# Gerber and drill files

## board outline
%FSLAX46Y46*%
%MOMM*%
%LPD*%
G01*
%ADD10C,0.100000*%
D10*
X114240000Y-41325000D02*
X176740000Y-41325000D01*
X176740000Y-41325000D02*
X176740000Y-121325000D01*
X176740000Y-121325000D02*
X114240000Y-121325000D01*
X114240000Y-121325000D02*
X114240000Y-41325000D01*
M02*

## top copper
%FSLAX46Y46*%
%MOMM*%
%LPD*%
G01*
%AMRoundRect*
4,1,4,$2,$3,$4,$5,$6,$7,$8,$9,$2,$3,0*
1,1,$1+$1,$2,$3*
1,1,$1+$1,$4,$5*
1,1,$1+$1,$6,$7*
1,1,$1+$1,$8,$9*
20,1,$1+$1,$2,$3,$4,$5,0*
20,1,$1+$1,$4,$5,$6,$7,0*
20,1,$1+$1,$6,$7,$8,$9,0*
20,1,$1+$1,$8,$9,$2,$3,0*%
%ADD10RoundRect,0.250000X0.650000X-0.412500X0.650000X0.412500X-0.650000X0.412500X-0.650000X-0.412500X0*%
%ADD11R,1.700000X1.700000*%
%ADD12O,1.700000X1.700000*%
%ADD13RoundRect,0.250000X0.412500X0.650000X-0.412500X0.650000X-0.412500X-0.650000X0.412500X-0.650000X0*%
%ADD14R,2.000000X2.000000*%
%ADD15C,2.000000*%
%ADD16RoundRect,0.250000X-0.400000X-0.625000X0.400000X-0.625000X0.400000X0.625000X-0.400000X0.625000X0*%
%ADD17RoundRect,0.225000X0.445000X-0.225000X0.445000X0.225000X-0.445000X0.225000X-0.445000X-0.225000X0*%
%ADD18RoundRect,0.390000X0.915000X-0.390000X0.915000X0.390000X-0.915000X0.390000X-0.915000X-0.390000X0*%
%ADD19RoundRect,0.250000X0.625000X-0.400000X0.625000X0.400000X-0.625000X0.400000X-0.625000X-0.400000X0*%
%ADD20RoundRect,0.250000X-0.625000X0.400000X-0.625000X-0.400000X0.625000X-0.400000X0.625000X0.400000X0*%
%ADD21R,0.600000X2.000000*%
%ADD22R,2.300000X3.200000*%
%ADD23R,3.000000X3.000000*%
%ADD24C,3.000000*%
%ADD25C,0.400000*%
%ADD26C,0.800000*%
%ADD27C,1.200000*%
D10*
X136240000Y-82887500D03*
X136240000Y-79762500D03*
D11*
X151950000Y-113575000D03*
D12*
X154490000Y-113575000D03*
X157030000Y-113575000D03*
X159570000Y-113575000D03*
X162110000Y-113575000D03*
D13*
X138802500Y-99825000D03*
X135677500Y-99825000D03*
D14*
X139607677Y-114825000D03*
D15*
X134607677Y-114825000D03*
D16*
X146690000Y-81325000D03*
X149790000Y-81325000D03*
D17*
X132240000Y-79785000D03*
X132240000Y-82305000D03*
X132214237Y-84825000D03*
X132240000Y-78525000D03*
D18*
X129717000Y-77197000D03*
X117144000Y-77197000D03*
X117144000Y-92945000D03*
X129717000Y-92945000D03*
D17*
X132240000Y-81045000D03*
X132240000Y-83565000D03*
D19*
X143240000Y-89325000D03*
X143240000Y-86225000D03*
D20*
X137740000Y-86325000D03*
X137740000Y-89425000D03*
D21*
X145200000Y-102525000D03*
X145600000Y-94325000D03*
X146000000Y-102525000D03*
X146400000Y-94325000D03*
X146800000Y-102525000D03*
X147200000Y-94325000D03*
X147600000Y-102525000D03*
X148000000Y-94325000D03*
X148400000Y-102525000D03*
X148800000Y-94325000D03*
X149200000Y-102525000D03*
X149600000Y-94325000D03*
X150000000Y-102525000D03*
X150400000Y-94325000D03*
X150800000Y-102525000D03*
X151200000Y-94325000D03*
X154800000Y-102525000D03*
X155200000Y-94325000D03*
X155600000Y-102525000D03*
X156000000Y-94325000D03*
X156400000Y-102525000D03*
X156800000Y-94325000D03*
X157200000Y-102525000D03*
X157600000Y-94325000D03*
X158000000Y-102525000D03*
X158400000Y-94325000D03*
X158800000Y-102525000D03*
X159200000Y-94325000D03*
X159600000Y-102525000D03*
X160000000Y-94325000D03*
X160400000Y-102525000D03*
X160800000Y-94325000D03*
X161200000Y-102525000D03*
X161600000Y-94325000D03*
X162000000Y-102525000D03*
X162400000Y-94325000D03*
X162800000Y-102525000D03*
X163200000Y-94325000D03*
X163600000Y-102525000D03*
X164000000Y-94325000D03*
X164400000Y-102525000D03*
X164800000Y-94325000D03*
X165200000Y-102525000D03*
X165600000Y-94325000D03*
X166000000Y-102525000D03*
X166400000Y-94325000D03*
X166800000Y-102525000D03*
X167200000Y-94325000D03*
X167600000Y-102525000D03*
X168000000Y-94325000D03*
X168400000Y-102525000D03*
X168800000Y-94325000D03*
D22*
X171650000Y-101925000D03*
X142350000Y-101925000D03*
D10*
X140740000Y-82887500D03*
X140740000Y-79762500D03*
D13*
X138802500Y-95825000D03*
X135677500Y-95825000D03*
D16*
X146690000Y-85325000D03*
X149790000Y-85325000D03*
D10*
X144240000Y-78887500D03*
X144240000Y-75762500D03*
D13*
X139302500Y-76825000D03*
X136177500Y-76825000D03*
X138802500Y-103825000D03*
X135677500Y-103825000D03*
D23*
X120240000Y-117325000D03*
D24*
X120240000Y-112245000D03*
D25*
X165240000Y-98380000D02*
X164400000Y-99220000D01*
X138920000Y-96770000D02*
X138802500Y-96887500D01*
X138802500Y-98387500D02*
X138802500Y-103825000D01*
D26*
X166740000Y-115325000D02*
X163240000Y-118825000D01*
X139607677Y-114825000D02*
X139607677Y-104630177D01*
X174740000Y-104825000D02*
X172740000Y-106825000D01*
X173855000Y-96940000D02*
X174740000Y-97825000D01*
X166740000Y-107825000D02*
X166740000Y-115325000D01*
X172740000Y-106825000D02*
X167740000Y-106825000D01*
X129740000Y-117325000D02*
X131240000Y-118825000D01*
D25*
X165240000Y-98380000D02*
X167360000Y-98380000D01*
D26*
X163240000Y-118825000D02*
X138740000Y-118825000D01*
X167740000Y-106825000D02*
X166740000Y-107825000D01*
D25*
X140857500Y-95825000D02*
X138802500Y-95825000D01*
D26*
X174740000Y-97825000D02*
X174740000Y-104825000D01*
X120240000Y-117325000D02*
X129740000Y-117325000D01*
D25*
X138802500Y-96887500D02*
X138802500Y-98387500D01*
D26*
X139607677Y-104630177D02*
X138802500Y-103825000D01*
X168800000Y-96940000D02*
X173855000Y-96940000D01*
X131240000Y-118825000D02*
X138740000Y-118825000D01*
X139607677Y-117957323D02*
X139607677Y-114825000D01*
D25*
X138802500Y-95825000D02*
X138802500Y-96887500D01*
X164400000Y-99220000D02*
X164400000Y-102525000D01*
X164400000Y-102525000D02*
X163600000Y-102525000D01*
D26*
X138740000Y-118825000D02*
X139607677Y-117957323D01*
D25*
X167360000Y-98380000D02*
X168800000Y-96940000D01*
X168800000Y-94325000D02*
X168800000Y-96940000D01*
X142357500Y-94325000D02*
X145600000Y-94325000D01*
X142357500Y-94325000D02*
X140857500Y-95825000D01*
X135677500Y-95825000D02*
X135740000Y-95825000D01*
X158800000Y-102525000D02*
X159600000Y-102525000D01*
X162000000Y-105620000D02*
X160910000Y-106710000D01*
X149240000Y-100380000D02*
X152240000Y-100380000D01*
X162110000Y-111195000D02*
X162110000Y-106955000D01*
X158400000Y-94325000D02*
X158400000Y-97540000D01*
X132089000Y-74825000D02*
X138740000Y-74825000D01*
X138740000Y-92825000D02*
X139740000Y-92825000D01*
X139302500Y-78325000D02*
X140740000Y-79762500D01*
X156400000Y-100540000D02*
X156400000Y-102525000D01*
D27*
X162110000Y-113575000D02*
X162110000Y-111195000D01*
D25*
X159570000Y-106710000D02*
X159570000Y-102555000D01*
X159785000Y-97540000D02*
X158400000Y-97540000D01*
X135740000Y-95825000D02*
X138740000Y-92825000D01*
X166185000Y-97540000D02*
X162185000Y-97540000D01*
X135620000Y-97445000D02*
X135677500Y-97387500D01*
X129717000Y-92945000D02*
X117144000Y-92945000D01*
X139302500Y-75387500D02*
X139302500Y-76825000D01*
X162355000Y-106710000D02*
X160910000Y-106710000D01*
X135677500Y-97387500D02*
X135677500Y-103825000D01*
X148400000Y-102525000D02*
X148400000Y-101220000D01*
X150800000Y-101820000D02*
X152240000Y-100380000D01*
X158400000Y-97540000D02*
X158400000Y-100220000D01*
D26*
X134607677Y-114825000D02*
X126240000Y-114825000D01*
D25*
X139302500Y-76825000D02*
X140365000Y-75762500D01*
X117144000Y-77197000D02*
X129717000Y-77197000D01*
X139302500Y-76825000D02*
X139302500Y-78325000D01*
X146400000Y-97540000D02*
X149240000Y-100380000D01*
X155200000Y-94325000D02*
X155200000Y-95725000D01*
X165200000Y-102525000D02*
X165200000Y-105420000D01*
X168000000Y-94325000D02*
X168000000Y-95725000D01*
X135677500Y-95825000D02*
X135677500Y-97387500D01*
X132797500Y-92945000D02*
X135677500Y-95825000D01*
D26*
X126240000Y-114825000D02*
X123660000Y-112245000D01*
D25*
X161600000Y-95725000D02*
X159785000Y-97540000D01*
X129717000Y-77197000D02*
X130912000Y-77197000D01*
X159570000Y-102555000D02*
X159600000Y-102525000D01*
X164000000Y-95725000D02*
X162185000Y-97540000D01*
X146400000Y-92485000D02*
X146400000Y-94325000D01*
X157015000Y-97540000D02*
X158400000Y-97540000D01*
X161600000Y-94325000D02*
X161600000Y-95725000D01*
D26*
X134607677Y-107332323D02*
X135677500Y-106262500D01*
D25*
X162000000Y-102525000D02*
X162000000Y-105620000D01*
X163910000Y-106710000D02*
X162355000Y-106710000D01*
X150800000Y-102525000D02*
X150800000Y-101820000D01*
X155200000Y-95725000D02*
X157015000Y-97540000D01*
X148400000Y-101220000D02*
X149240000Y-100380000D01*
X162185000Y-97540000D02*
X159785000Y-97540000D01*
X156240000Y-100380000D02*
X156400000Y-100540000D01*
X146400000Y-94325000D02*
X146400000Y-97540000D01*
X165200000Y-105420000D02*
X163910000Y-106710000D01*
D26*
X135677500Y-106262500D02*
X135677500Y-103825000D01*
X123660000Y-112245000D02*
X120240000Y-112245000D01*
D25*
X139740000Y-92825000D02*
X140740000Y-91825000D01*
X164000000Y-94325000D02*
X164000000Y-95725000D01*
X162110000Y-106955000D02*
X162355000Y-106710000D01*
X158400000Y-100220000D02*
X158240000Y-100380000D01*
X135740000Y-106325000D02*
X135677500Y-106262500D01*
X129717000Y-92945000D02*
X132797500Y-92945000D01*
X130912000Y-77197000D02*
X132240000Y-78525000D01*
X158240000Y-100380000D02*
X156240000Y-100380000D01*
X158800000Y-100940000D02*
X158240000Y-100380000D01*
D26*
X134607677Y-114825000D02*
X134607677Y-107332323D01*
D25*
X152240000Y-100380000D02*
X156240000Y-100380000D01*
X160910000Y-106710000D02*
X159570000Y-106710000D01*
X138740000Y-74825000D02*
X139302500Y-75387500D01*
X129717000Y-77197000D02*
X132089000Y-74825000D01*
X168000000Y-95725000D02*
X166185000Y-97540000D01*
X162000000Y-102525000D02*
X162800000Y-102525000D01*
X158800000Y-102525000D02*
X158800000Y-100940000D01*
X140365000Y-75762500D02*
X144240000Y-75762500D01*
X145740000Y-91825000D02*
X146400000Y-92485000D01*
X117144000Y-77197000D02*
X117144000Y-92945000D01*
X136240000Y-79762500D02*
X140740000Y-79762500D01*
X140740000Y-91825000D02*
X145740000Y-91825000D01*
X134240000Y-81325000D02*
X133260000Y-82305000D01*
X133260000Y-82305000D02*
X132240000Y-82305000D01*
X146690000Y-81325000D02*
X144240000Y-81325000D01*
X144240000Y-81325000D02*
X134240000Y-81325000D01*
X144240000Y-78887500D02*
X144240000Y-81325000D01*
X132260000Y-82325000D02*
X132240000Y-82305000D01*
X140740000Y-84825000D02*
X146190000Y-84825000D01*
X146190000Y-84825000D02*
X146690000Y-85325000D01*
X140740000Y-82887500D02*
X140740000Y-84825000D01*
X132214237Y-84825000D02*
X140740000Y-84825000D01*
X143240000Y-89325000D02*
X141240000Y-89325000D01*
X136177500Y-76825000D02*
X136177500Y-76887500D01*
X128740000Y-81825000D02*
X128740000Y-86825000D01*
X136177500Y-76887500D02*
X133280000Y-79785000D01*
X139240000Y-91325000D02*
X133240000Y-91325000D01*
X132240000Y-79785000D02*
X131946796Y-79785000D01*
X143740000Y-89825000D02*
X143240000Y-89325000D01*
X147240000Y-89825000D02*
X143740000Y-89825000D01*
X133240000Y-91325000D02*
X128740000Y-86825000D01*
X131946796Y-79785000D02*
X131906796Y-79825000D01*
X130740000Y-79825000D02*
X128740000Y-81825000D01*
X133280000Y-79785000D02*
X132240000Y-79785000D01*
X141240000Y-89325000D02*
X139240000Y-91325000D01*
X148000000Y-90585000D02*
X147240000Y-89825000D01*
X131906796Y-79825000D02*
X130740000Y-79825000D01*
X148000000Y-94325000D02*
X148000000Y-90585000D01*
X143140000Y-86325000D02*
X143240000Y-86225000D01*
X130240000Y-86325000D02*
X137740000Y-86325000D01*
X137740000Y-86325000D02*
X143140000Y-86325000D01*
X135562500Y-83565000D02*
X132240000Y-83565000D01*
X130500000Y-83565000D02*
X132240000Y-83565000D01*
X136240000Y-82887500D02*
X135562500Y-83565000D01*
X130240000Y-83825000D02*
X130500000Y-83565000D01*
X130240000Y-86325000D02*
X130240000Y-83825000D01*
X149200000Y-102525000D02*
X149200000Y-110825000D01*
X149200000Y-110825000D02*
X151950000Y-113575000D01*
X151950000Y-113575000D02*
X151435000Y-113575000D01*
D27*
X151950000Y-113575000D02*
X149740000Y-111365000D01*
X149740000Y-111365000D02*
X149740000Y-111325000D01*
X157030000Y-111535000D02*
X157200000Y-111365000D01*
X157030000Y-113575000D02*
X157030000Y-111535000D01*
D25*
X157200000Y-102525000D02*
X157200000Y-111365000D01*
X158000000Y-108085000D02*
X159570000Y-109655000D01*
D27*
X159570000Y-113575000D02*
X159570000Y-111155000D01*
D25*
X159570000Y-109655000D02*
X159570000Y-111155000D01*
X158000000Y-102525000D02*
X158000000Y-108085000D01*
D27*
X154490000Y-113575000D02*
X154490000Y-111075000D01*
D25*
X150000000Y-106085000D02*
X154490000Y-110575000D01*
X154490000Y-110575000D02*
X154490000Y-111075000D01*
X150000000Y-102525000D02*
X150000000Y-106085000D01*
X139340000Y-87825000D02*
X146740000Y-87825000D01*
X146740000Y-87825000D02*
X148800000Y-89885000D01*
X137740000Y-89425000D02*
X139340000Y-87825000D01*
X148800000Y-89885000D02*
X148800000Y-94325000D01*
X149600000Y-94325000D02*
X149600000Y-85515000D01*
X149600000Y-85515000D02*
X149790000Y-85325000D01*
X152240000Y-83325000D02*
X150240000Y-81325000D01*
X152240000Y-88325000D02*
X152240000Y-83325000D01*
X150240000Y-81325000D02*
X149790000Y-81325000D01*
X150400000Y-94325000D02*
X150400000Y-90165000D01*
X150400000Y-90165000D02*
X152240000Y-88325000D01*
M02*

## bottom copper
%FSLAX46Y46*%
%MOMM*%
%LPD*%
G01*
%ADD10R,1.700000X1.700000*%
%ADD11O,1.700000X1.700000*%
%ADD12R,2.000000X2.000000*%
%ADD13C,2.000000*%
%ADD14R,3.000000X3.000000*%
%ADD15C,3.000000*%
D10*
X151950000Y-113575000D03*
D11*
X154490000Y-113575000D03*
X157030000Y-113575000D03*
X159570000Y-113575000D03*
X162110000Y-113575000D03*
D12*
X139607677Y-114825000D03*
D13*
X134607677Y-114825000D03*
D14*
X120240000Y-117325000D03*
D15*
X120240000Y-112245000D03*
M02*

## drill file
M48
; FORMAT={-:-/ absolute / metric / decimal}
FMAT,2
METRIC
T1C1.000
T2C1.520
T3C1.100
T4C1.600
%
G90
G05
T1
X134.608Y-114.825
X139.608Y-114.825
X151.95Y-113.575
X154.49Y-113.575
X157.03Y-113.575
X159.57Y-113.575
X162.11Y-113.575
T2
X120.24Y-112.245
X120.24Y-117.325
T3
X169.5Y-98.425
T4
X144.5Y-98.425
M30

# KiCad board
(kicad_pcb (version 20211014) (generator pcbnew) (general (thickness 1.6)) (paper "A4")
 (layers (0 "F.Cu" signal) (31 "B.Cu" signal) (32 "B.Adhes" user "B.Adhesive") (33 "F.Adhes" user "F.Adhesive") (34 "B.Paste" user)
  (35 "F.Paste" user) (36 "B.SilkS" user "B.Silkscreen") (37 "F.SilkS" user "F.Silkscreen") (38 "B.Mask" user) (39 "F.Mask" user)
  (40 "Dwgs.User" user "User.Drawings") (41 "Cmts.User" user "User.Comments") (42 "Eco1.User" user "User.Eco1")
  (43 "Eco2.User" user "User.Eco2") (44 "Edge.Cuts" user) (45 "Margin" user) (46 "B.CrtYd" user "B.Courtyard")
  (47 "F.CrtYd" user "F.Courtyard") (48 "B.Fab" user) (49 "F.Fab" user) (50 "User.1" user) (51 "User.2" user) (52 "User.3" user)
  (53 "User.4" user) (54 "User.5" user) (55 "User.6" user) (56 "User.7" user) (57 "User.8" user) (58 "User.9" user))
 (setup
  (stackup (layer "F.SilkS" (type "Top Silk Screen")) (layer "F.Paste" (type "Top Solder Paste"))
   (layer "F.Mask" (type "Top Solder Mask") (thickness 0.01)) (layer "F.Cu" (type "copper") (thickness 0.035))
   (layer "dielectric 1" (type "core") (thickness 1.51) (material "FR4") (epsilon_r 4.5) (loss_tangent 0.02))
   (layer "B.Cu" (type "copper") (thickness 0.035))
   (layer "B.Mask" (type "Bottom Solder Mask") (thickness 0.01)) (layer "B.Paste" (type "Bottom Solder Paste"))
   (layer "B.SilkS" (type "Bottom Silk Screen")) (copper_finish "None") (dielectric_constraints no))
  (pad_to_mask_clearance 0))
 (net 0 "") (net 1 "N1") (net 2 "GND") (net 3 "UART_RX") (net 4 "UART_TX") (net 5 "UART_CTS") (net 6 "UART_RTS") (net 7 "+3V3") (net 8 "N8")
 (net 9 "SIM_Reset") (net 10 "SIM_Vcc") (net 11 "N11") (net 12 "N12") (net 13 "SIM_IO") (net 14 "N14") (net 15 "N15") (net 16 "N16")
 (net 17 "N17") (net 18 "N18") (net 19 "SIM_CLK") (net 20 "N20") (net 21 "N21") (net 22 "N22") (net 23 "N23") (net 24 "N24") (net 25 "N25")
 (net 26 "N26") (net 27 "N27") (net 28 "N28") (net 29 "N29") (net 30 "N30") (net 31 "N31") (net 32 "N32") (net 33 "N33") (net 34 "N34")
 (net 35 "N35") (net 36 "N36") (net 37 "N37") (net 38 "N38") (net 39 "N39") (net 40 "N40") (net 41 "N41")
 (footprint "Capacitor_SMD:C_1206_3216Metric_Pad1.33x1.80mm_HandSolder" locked (layer "F.Cu") (at 136.24 81.325 90)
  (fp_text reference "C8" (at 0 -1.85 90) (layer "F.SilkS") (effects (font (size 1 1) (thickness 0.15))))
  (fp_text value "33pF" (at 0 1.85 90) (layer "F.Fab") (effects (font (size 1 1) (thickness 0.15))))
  (pad "1" smd roundrect locked (at -1.5625 0 90) (size 1.325 1.8) (layers "F.Cu" "F.Paste" "F.Mask") (roundrect_rratio 0.188679)
   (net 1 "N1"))
  (pad "2" smd roundrect locked (at 1.5625 0 90) (size 1.325 1.8) (layers "F.Cu" "F.Paste" "F.Mask") (roundrect_rratio 0.188679)
   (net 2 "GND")))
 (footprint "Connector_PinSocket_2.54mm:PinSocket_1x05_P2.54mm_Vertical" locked (layer "F.Cu") (at 151.95 113.575 90)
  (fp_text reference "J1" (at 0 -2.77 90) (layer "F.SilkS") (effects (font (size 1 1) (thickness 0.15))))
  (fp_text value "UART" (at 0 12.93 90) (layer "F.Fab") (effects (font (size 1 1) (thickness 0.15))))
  (pad "1" thru_hole rect locked (at 0 0 90) (size 1.7 1.7) (drill 1) (layers *.Cu *.Mask) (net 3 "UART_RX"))
  (pad "2" thru_hole oval locked (at 0 2.54 90) (size 1.7 1.7) (drill 1) (layers *.Cu *.Mask) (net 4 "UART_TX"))
  (pad "3" thru_hole oval locked (at 0 5.08 90) (size 1.7 1.7) (drill 1) (layers *.Cu *.Mask) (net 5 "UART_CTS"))
  (pad "4" thru_hole oval locked (at 0 7.62 90) (size 1.7 1.7) (drill 1) (layers *.Cu *.Mask) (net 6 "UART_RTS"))
  (pad "5" thru_hole oval locked (at 0 10.16 90) (size 1.7 1.7) (drill 1) (layers *.Cu *.Mask) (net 2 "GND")))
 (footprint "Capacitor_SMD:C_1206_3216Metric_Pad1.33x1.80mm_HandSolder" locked (layer "F.Cu") (at 137.24 99.825 180)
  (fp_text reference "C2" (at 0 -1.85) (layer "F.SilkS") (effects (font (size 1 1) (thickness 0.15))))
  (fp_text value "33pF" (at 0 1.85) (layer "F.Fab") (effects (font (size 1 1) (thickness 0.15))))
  (pad "1" smd roundrect locked (at -1.5625 0 180) (size 1.325 1.8) (layers "F.Cu" "F.Paste" "F.Mask") (roundrect_rratio 0.188679)
   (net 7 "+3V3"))
  (pad "2" smd roundrect locked (at 1.5625 0 180) (size 1.325 1.8) (layers "F.Cu" "F.Paste" "F.Mask") (roundrect_rratio 0.188679)
   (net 2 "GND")))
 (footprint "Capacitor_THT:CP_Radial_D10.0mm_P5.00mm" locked (layer "F.Cu") (at 139.607677 114.825 180)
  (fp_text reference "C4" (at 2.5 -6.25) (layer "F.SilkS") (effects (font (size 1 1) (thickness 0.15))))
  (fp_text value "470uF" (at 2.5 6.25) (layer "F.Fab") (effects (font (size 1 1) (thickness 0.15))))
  (pad "1" thru_hole rect locked (at 0 0 180) (size 2 2) (drill 1) (layers *.Cu *.Mask) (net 7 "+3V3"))
  (pad "2" thru_hole circle locked (at 5 0 180) (size 2 2) (drill 1) (layers *.Cu *.Mask) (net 2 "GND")))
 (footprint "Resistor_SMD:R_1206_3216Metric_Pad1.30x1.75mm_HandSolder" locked (layer "F.Cu") (at 148.24 81.325)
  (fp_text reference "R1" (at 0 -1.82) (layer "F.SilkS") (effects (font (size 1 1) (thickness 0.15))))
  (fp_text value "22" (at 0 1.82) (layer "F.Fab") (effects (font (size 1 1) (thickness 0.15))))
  (pad "1" smd roundrect locked (at -1.55 0) (size 1.3 1.75) (layers "F.Cu" "F.Paste" "F.Mask") (roundrect_rratio 0.192308) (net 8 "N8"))
  (pad "2" smd roundrect locked (at 1.55 0) (size 1.3 1.75) (layers "F.Cu" "F.Paste" "F.Mask") (roundrect_rratio 0.192308)
   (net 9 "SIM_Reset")))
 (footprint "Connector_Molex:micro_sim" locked (layer "F.Cu") (at 123.24 85.325 -90)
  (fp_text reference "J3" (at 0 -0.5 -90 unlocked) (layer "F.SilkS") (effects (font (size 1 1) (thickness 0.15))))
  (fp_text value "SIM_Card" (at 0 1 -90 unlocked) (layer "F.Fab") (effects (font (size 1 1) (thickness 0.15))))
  (pad "1" smd roundrect locked (at -5.54 -9 90) (size 0.9 1.34) (layers "F.Cu" "F.Paste" "F.Mask") (roundrect_rratio 0.25)
   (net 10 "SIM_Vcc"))
  (pad "2" smd roundrect locked (at -3.02 -9 90) (size 0.9 1.34) (layers "F.Cu" "F.Paste" "F.Mask") (roundrect_rratio 0.25) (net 8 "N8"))
  (pad "3" smd roundrect locked (at -0.5 -8.974237 90) (size 0.9 1.34) (layers "F.Cu" "F.Paste" "F.Mask") (roundrect_rratio 0.25)
   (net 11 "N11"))
  (pad "5" smd roundrect locked (at -6.8 -9 90) (size 0.9 1.34) (layers "F.Cu" "F.Paste" "F.Mask") (roundrect_rratio 0.25) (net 2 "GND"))
  (pad "5" smd roundrect locked (at -8.128 -6.477 90) (size 1.56 2.61) (layers "F.Cu" "F.Paste" "F.Mask") (roundrect_rratio 0.25)
   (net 2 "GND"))
  (pad "5" smd roundrect locked (at -8.128 6.096 90) (size 1.56 2.61) (layers "F.Cu" "F.Paste" "F.Mask") (roundrect_rratio 0.25)
   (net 2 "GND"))
  (pad "5" smd roundrect locked (at 7.62 6.096 90) (size 1.56 2.61) (layers "F.Cu" "F.Paste" "F.Mask") (roundrect_rratio 0.25) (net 2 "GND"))
  (pad "5" smd roundrect locked (at 7.62 -6.477 90) (size 1.56 2.61) (layers "F.Cu" "F.Paste" "F.Mask") (roundrect_rratio 0.25)
   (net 2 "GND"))
  (pad "6" smd roundrect locked (at -4.28 -9 90) (size 0.9 1.34) (layers "F.Cu" "F.Paste" "F.Mask") (roundrect_rratio 0.25) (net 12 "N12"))
  (pad "7" smd roundrect locked (at -1.76 -9 90) (size 0.9 1.34) (layers "F.Cu" "F.Paste" "F.Mask") (roundrect_rratio 0.25) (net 1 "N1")))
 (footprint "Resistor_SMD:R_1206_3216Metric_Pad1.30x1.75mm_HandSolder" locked (layer "F.Cu") (at 143.24 87.775 90)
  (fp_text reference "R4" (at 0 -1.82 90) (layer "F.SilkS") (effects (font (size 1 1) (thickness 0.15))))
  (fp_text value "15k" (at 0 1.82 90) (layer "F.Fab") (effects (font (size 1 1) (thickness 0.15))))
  (pad "1" smd roundrect locked (at -1.55 0 90) (size 1.3 1.75) (layers "F.Cu" "F.Paste" "F.Mask") (roundrect_rratio 0.192308)
   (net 10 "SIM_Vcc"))
  (pad "2" smd roundrect locked (at 1.55 0 90) (size 1.3 1.75) (layers "F.Cu" "F.Paste" "F.Mask") (roundrect_rratio 0.192308) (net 1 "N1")))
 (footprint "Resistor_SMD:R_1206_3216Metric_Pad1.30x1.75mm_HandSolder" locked (layer "F.Cu") (at 137.74 87.875 -90)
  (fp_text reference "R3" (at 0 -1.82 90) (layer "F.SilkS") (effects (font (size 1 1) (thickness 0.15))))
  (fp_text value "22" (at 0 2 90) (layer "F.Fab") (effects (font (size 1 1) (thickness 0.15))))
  (pad "1" smd roundrect locked (at -1.55 0 270) (size 1.3 1.75) (layers "F.Cu" "F.Paste" "F.Mask") (roundrect_rratio 0.192308) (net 1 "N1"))
  (pad "2" smd roundrect locked (at 1.55 0 270) (size 1.3 1.75) (layers "F.Cu" "F.Paste" "F.Mask") (roundrect_rratio 0.192308)
   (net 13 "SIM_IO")))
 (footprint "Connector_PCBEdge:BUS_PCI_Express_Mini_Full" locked (layer "F.Cu") (at 157 98.425)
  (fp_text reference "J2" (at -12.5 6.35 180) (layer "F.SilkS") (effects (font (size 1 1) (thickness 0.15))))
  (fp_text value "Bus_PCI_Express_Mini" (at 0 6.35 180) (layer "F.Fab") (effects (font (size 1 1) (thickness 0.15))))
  (pad "" np_thru_hole circle locked (at -12.5 0) (size 1.6 1.6) (drill 1.6) (layers *.Cu *.Mask))
  (pad "" np_thru_hole circle locked (at 12.5 0) (size 1.1 1.1) (drill 1.1) (layers *.Cu *.Mask))
  (pad "1" smd rect locked (at -11.8 4.1) (size 0.6 2) (layers "F.Cu" "F.Paste" "F.Mask") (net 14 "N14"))
  (pad "2" smd rect locked (at -11.4 -4.1) (size 0.6 2) (layers "F.Cu" "F.Paste" "F.Mask") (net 7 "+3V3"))
  (pad "3" smd rect locked (at -11 4.1) (size 0.6 2) (layers "F.Cu" "F.Paste" "F.Mask") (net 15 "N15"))
  (pad "4" smd rect locked (at -10.6 -4.1) (size 0.6 2) (layers "F.Cu" "F.Paste" "F.Mask") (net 2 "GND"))
  (pad "5" smd rect locked (at -10.2 4.1) (size 0.6 2) (layers "F.Cu" "F.Paste" "F.Mask") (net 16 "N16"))
  (pad "6" smd rect locked (at -9.8 -4.1) (size 0.6 2) (layers "F.Cu" "F.Paste" "F.Mask") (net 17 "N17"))
  (pad "7" smd rect locked (at -9.4 4.1) (size 0.6 2) (layers "F.Cu" "F.Paste" "F.Mask") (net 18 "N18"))
  (pad "8" smd rect locked (at -9 -4.1) (size 0.6 2) (layers "F.Cu" "F.Paste" "F.Mask") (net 10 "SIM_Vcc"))
  (pad "9" smd rect locked (at -8.6 4.1) (size 0.6 2) (layers "F.Cu" "F.Paste" "F.Mask") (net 2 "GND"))
  (pad "10" smd rect locked (at -8.2 -4.1) (size 0.6 2) (layers "F.Cu" "F.Paste" "F.Mask") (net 13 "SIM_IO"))
  (pad "11" smd rect locked (at -7.8 4.1) (size 0.6 2) (layers "F.Cu" "F.Paste" "F.Mask") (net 3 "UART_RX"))
  (pad "12" smd rect locked (at -7.4 -4.1) (size 0.6 2) (layers "F.Cu" "F.Paste" "F.Mask") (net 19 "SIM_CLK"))
  (pad "13" smd rect locked (at -7 4.1) (size 0.6 2) (layers "F.Cu" "F.Paste" "F.Mask") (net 4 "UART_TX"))
  (pad "14" smd rect locked (at -6.6 -4.1) (size 0.6 2) (layers "F.Cu" "F.Paste" "F.Mask") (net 9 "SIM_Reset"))
  (pad "15" smd rect locked (at -6.2 4.1) (size 0.6 2) (layers "F.Cu" "F.Paste" "F.Mask") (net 2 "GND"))
  (pad "16" smd rect locked (at -5.8 -4.1) (size 0.6 2) (layers "F.Cu" "F.Paste" "F.Mask") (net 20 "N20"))
  (pad "17" smd rect locked (at -2.2 4.1) (size 0.6 2) (layers "F.Cu" "F.Paste" "F.Mask") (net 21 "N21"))
  (pad "18" smd rect locked (at -1.8 -4.1) (size 0.6 2) (layers "F.Cu" "F.Paste" "F.Mask") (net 2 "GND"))
  (pad "19" smd rect locked (at -1.4 4.1) (size 0.6 2) (layers "F.Cu" "F.Paste" "F.Mask") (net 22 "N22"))
  (pad "20" smd rect locked (at -1 -4.1) (size 0.6 2) (layers "F.Cu" "F.Paste" "F.Mask") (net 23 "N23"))
  (pad "21" smd rect locked (at -0.6 4.1) (size 0.6 2) (layers "F.Cu" "F.Paste" "F.Mask") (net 2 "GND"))
  (pad "22" smd rect locked (at -0.2 -4.1) (size 0.6 2) (layers "F.Cu" "F.Paste" "F.Mask") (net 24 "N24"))
  (pad "23" smd rect locked (at 0.2 4.1) (size 0.6 2) (layers "F.Cu" "F.Paste" "F.Mask") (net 5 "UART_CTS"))
  (pad "24" smd rect locked (at 0.6 -4.1) (size 0.6 2) (layers "F.Cu" "F.Paste" "F.Mask") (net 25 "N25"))
  (pad "25" smd rect locked (at 1 4.1) (size 0.6 2) (layers "F.Cu" "F.Paste" "F.Mask") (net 6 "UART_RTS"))
  (pad "26" smd rect locked (at 1.4 -4.1) (size 0.6 2) (layers "F.Cu" "F.Paste" "F.Mask") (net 2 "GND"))
  (pad "27" smd rect locked (at 1.8 4.1) (size 0.6 2) (layers "F.Cu" "F.Paste" "F.Mask") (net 2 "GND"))
  (pad "28" smd rect locked (at 2.2 -4.1) (size 0.6 2) (layers "F.Cu" "F.Paste" "F.Mask") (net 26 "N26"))
  (pad "29" smd rect locked (at 2.6 4.1) (size 0.6 2) (layers "F.Cu" "F.Paste" "F.Mask") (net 2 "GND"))
  (pad "30" smd rect locked (at 3 -4.1) (size 0.6 2) (layers "F.Cu" "F.Paste" "F.Mask") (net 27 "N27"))
  (pad "31" smd rect locked (at 3.4 4.1) (size 0.6 2) (layers "F.Cu" "F.Paste" "F.Mask") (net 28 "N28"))
  (pad "32" smd rect locked (at 3.8 -4.1) (size 0.6 2) (layers "F.Cu" "F.Paste" "F.Mask") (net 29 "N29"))
  (pad "33" smd rect locked (at 4.2 4.1) (size 0.6 2) (layers "F.Cu" "F.Paste" "F.Mask") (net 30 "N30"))
  (pad "34" smd rect locked (at 4.6 -4.1) (size 0.6 2) (layers "F.Cu" "F.Paste" "F.Mask") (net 2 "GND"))
  (pad "35" smd rect locked (at 5 4.1) (size 0.6 2) (layers "F.Cu" "F.Paste" "F.Mask") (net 2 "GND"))
  (pad "36" smd rect locked (at 5.4 -4.1) (size 0.6 2) (layers "F.Cu" "F.Paste" "F.Mask") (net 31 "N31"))
  (pad "37" smd rect locked (at 5.8 4.1) (size 0.6 2) (layers "F.Cu" "F.Paste" "F.Mask") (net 2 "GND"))
  (pad "38" smd rect locked (at 6.2 -4.1) (size 0.6 2) (layers "F.Cu" "F.Paste" "F.Mask") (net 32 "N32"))
  (pad "39" smd rect locked (at 6.6 4.1) (size 0.6 2) (layers "F.Cu" "F.Paste" "F.Mask") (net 7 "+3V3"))
  (pad "40" smd rect locked (at 7 -4.1) (size 0.6 2) (layers "F.Cu" "F.Paste" "F.Mask") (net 2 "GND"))
  (pad "41" smd rect locked (at 7.4 4.1) (size 0.6 2) (layers "F.Cu" "F.Paste" "F.Mask") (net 7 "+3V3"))
  (pad "42" smd rect locked (at 7.8 -4.1) (size 0.6 2) (layers "F.Cu" "F.Paste" "F.Mask") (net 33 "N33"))
  (pad "43" smd rect locked (at 8.2 4.1) (size 0.6 2) (layers "F.Cu" "F.Paste" "F.Mask") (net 2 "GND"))
  (pad "44" smd rect locked (at 8.6 -4.1) (size 0.6 2) (layers "F.Cu" "F.Paste" "F.Mask") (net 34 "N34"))
  (pad "45" smd rect locked (at 9 4.1) (size 0.6 2) (layers "F.Cu" "F.Paste" "F.Mask") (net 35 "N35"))
  (pad "46" smd rect locked (at 9.4 -4.1) (size 0.6 2) (layers "F.Cu" "F.Paste" "F.Mask") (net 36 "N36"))
  (pad "47" smd rect locked (at 9.8 4.1) (size 0.6 2) (layers "F.Cu" "F.Paste" "F.Mask") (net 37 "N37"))
  (pad "48" smd rect locked (at 10.2 -4.1) (size 0.6 2) (layers "F.Cu" "F.Paste" "F.Mask") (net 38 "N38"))
  (pad "49" smd rect locked (at 10.6 4.1) (size 0.6 2) (layers "F.Cu" "F.Paste" "F.Mask") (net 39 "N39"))
  (pad "50" smd rect locked (at 11 -4.1) (size 0.6 2) (layers "F.Cu" "F.Paste" "F.Mask") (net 2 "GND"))
  (pad "51" smd rect locked (at 11.4 4.1) (size 0.6 2) (layers "F.Cu" "F.Paste" "F.Mask") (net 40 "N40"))
  (pad "52" smd rect locked (at 11.8 -4.1) (size 0.6 2) (layers "F.Cu" "F.Paste" "F.Mask") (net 7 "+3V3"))
  (pad "MP" smd rect locked (at 14.65 3.5) (size 2.3 3.2) (layers "F.Cu" "F.Paste" "F.Mask") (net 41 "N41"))
  (pad "MP" smd rect locked (at -14.65 3.5) (size 2.3 3.2) (layers "F.Cu" "F.Paste" "F.Mask") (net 41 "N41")))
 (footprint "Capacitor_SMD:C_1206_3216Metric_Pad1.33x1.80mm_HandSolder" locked (layer "F.Cu") (at 140.74 81.325 90)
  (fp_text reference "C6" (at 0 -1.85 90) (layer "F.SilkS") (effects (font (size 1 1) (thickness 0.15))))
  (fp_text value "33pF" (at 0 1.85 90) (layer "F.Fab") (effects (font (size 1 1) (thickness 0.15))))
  (pad "1" smd roundrect locked (at -1.5625 0 90) (size 1.325 1.8) (layers "F.Cu" "F.Paste" "F.Mask") (roundrect_rratio 0.188679)
   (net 11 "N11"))
  (pad "2" smd roundrect locked (at 1.5625 0 90) (size 1.325 1.8) (layers "F.Cu" "F.Paste" "F.Mask") (roundrect_rratio 0.188679)
   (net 2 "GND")))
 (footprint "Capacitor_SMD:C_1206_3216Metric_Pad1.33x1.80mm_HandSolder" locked (layer "F.Cu") (at 137.24 95.825 180)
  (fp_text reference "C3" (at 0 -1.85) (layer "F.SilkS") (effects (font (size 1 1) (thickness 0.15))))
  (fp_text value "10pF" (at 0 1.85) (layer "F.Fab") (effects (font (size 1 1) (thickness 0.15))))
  (pad "1" smd roundrect locked (at -1.5625 0 180) (size 1.325 1.8) (layers "F.Cu" "F.Paste" "F.Mask") (roundrect_rratio 0.188679)
   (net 7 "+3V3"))
  (pad "2" smd roundrect locked (at 1.5625 0 180) (size 1.325 1.8) (layers "F.Cu" "F.Paste" "F.Mask") (roundrect_rratio 0.188679)
   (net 2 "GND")))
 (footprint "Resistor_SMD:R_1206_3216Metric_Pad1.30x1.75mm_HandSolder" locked (layer "F.Cu") (at 148.24 85.325)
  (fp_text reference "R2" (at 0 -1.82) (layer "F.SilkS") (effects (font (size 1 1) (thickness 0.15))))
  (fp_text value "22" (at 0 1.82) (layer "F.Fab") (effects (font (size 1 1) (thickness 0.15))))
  (pad "1" smd roundrect locked (at -1.55 0) (size 1.3 1.75) (layers "F.Cu" "F.Paste" "F.Mask") (roundrect_rratio 0.192308) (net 11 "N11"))
  (pad "2" smd roundrect locked (at 1.55 0) (size 1.3 1.75) (layers "F.Cu" "F.Paste" "F.Mask") (roundrect_rratio 0.192308)
   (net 19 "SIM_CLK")))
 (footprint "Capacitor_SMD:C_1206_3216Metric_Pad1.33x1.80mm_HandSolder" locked (layer "F.Cu") (at 144.24 77.325 90)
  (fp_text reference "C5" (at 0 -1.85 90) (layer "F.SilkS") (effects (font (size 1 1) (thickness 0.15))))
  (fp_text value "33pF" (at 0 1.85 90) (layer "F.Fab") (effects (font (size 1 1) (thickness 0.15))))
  (pad "1" smd roundrect locked (at -1.5625 0 90) (size 1.325 1.8) (layers "F.Cu" "F.Paste" "F.Mask") (roundrect_rratio 0.188679)
   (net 8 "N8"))
  (pad "2" smd roundrect locked (at 1.5625 0 90) (size 1.325 1.8) (layers "F.Cu" "F.Paste" "F.Mask") (roundrect_rratio 0.188679)
   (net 2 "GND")))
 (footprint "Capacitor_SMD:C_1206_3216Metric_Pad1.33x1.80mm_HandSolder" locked (layer "F.Cu") (at 137.74 76.825 180)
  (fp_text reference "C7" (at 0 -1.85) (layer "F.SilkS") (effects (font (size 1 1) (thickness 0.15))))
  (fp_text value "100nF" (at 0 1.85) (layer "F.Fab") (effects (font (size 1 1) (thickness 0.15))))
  (pad "1" smd roundrect locked (at -1.5625 0 180) (size 1.325 1.8) (layers "F.Cu" "F.Paste" "F.Mask") (roundrect_rratio 0.188679)
   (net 2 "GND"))
  (pad "2" smd roundrect locked (at 1.5625 0 180) (size 1.325 1.8) (layers "F.Cu" "F.Paste" "F.Mask") (roundrect_rratio 0.188679)
   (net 10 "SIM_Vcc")))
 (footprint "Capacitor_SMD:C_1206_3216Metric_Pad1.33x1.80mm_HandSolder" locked (layer "F.Cu") (at 137.24 103.825 180)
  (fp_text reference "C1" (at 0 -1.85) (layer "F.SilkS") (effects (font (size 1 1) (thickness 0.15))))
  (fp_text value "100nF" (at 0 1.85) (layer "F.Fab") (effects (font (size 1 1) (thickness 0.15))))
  (pad "1" smd roundrect locked (at -1.5625 0 180) (size 1.325 1.8) (layers "F.Cu" "F.Paste" "F.Mask") (roundrect_rratio 0.188679)
   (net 7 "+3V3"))
  (pad "2" smd roundrect locked (at 1.5625 0 180) (size 1.325 1.8) (layers "F.Cu" "F.Paste" "F.Mask") (roundrect_rratio 0.188679)
   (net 2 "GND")))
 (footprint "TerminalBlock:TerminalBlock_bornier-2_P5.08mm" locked (layer "F.Cu") (at 120.24 117.325 90)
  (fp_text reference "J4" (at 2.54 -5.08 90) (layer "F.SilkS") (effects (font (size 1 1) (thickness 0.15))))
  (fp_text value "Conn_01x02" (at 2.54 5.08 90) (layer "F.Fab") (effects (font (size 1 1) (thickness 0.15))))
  (pad "1" thru_hole rect locked (at 0 0 90) (size 3 3) (drill 1.52) (layers *.Cu *.Mask) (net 7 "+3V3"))
  (pad "2" thru_hole circle locked (at 5.08 0 90) (size 3 3) (drill 1.52) (layers *.Cu *.Mask) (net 2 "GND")))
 (gr_line locked (start 114.24 41.325) (end 176.74 41.325) (layer "Edge.Cuts") (width 0.1))
 (gr_line locked (start 176.74 41.325) (end 176.74 121.325) (layer "Edge.Cuts") (width 0.1))
 (gr_line locked (start 176.74 121.325) (end 114.24 121.325) (layer "Edge.Cuts") (width 0.1))
 (gr_line locked (start 114.24 121.325) (end 114.24 41.325) (layer "Edge.Cuts") (width 0.1))
 (segment locked (start 165.24 98.38) (end 164.4 99.22) (width 0.4) (layer "F.Cu") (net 7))
 (segment locked (start 138.92 96.77) (end 138.8025 96.8875) (width 0.4) (layer "F.Cu") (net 7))
 (segment locked (start 138.8025 98.3875) (end 138.8025 103.825) (width 0.4) (layer "F.Cu") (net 7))
 (segment locked (start 166.74 115.325) (end 163.24 118.825) (width 0.8) (layer "F.Cu") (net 7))
 (segment locked (start 139.607677 114.825) (end 139.607677 104.630177) (width 0.8) (layer "F.Cu") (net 7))
 (segment locked (start 174.74 104.825) (end 172.74 106.825) (width 0.8) (layer "F.Cu") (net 7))
 (segment locked (start 173.855 96.94) (end 174.74 97.825) (width 0.8) (layer "F.Cu") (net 7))
 (segment locked (start 166.74 107.825) (end 166.74 115.325) (width 0.8) (layer "F.Cu") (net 7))
 (segment locked (start 172.74 106.825) (end 167.74 106.825) (width 0.8) (layer "F.Cu") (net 7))
 (segment locked (start 129.74 117.325) (end 131.24 118.825) (width 0.8) (layer "F.Cu") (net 7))
 (segment locked (start 165.24 98.38) (end 167.36 98.38) (width 0.4) (layer "F.Cu") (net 7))
 (segment locked (start 163.24 118.825) (end 138.74 118.825) (width 0.8) (layer "F.Cu") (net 7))
 (segment locked (start 167.74 106.825) (end 166.74 107.825) (width 0.8) (layer "F.Cu") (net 7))
 (segment locked (start 140.8575 95.825) (end 138.8025 95.825) (width 0.4) (layer "F.Cu") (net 7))
 (segment locked (start 174.74 97.825) (end 174.74 104.825) (width 0.8) (layer "F.Cu") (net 7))
 (segment locked (start 120.24 117.325) (end 129.74 117.325) (width 0.8) (layer "F.Cu") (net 7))
 (segment locked (start 138.8025 96.8875) (end 138.8025 98.3875) (width 0.4) (layer "F.Cu") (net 7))
 (segment locked (start 139.607677 104.630177) (end 138.8025 103.825) (width 0.8) (layer "F.Cu") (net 7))
 (segment locked (start 168.8 96.94) (end 173.855 96.94) (width 0.8) (layer "F.Cu") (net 7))
 (segment locked (start 131.24 118.825) (end 138.74 118.825) (width 0.8) (layer "F.Cu") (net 7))
 (segment locked (start 139.607677 117.957323) (end 139.607677 114.825) (width 0.8) (layer "F.Cu") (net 7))
 (segment locked (start 138.8025 95.825) (end 138.8025 96.8875) (width 0.4) (layer "F.Cu") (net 7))
 (segment locked (start 164.4 99.22) (end 164.4 102.525) (width 0.4) (layer "F.Cu") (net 7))
 (segment locked (start 164.4 102.525) (end 163.6 102.525) (width 0.4) (layer "F.Cu") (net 7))
 (segment locked (start 138.74 118.825) (end 139.607677 117.957323) (width 0.8) (layer "F.Cu") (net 7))
 (segment locked (start 167.36 98.38) (end 168.8 96.94) (width 0.4) (layer "F.Cu") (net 7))
 (segment locked (start 168.8 94.325) (end 168.8 96.94) (width 0.4) (layer "F.Cu") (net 7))
 (segment locked (start 142.3575 94.325) (end 145.6 94.325) (width 0.4) (layer "F.Cu") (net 7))
 (segment locked (start 142.3575 94.325) (end 140.8575 95.825) (width 0.4) (layer "F.Cu") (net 7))
 (segment locked (start 135.6775 95.825) (end 135.74 95.825) (width 0.4) (layer "F.Cu") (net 2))
 (segment locked (start 158.8 102.525) (end 159.6 102.525) (width 0.4) (layer "F.Cu") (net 2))
 (segment locked (start 162 105.62) (end 160.91 106.71) (width 0.4) (layer "F.Cu") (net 2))
 (segment locked (start 149.24 100.38) (end 152.24 100.38) (width 0.4) (layer "F.Cu") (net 2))
 (segment locked (start 162.11 111.195) (end 162.11 106.955) (width 0.4) (layer "F.Cu") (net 2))
 (segment locked (start 158.4 94.325) (end 158.4 97.54) (width 0.4) (layer "F.Cu") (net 2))
 (segment locked (start 132.089 74.825) (end 138.74 74.825) (width 0.4) (layer "F.Cu") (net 2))
 (segment locked (start 138.74 92.825) (end 139.74 92.825) (width 0.4) (layer "F.Cu") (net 2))
 (segment locked (start 139.3025 78.325) (end 140.74 79.7625) (width 0.4) (layer "F.Cu") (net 2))
 (segment locked (start 156.4 100.54) (end 156.4 102.525) (width 0.4) (layer "F.Cu") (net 2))
 (segment locked (start 162.11 113.575) (end 162.11 111.195) (width 1.2) (layer "F.Cu") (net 2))
 (segment locked (start 159.57 106.71) (end 159.57 102.555) (width 0.4) (layer "F.Cu") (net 2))
 (segment locked (start 159.785 97.54) (end 158.4 97.54) (width 0.4) (layer "F.Cu") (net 2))
 (segment locked (start 135.74 95.825) (end 138.74 92.825) (width 0.4) (layer "F.Cu") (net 2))
 (segment locked (start 166.185 97.54) (end 162.185 97.54) (width 0.4) (layer "F.Cu") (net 2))
 (segment locked (start 135.62 97.445) (end 135.6775 97.3875) (width 0.4) (layer "F.Cu") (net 2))
 (segment locked (start 129.717 92.945) (end 117.144 92.945) (width 0.4) (layer "F.Cu") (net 2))
 (segment locked (start 139.3025 75.3875) (end 139.3025 76.825) (width 0.4) (layer "F.Cu") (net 2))
 (segment locked (start 162.355 106.71) (end 160.91 106.71) (width 0.4) (layer "F.Cu") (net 2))
 (segment locked (start 135.6775 97.3875) (end 135.6775 103.825) (width 0.4) (layer "F.Cu") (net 2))
 (segment locked (start 148.4 102.525) (end 148.4 101.22) (width 0.4) (layer "F.Cu") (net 2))
 (segment locked (start 150.8 101.82) (end 152.24 100.38) (width 0.4) (layer "F.Cu") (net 2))
 (segment locked (start 158.4 97.54) (end 158.4 100.22) (width 0.4) (layer "F.Cu") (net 2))
 (segment locked (start 134.607677 114.825) (end 126.24 114.825) (width 0.8) (layer "F.Cu") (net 2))
 (segment locked (start 139.3025 76.825) (end 140.365 75.7625) (width 0.4) (layer "F.Cu") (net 2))
 (segment locked (start 117.144 77.197) (end 129.717 77.197) (width 0.4) (layer "F.Cu") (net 2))
 (segment locked (start 139.3025 76.825) (end 139.3025 78.325) (width 0.4) (layer "F.Cu") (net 2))
 (segment locked (start 146.4 97.54) (end 149.24 100.38) (width 0.4) (layer "F.Cu") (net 2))
 (segment locked (start 155.2 94.325) (end 155.2 95.725) (width 0.4) (layer "F.Cu") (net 2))
 (segment locked (start 165.2 102.525) (end 165.2 105.42) (width 0.4) (layer "F.Cu") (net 2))
 (segment locked (start 168 94.325) (end 168 95.725) (width 0.4) (layer "F.Cu") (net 2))
 (segment locked (start 135.6775 95.825) (end 135.6775 97.3875) (width 0.4) (layer "F.Cu") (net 2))
 (segment locked (start 132.7975 92.945) (end 135.6775 95.825) (width 0.4) (layer "F.Cu") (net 2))
 (segment locked (start 126.24 114.825) (end 123.66 112.245) (width 0.8) (layer "F.Cu") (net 2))
 (segment locked (start 161.6 95.725) (end 159.785 97.54) (width 0.4) (layer "F.Cu") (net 2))
 (segment locked (start 129.717 77.197) (end 130.912 77.197) (width 0.4) (layer "F.Cu") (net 2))
 (segment locked (start 159.57 102.555) (end 159.6 102.525) (width 0.4) (layer "F.Cu") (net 2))
 (segment locked (start 164 95.725) (end 162.185 97.54) (width 0.4) (layer "F.Cu") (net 2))
 (segment locked (start 146.4 92.485) (end 146.4 94.325) (width 0.4) (layer "F.Cu") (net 2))
 (segment locked (start 157.015 97.54) (end 158.4 97.54) (width 0.4) (layer "F.Cu") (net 2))
 (segment locked (start 161.6 94.325) (end 161.6 95.725) (width 0.4) (layer "F.Cu") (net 2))
 (segment locked (start 134.607677 107.332323) (end 135.6775 106.2625) (width 0.8) (layer "F.Cu") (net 2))
 (segment locked (start 162 102.525) (end 162 105.62) (width 0.4) (layer "F.Cu") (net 2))
 (segment locked (start 163.91 106.71) (end 162.355 106.71) (width 0.4) (layer "F.Cu") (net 2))
 (segment locked (start 150.8 102.525) (end 150.8 101.82) (width 0.4) (layer "F.Cu") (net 2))
 (segment locked (start 155.2 95.725) (end 157.015 97.54) (width 0.4) (layer "F.Cu") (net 2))
 (segment locked (start 148.4 101.22) (end 149.24 100.38) (width 0.4) (layer "F.Cu") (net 2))
 (segment locked (start 162.185 97.54) (end 159.785 97.54) (width 0.4) (layer "F.Cu") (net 2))
 (segment locked (start 156.24 100.38) (end 156.4 100.54) (width 0.4) (layer "F.Cu") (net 2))
 (segment locked (start 146.4 94.325) (end 146.4 97.54) (width 0.4) (layer "F.Cu") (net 2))
 (segment locked (start 165.2 105.42) (end 163.91 106.71) (width 0.4) (layer "F.Cu") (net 2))
 (segment locked (start 135.6775 106.2625) (end 135.6775 103.825) (width 0.8) (layer "F.Cu") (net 2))
 (segment locked (start 123.66 112.245) (end 120.24 112.245) (width 0.8) (layer "F.Cu") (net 2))
 (segment locked (start 139.74 92.825) (end 140.74 91.825) (width 0.4) (layer "F.Cu") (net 2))
 (segment locked (start 164 94.325) (end 164 95.725) (width 0.4) (layer "F.Cu") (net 2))
 (segment locked (start 162.11 106.955) (end 162.355 106.71) (width 0.4) (layer "F.Cu") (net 2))
 (segment locked (start 158.4 100.22) (end 158.24 100.38) (width 0.4) (layer "F.Cu") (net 2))
 (segment locked (start 135.74 106.325) (end 135.6775 106.2625) (width 0.4) (layer "F.Cu") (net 2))
 (segment locked (start 129.717 92.945) (end 132.7975 92.945) (width 0.4) (layer "F.Cu") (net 2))
 (segment locked (start 130.912 77.197) (end 132.24 78.525) (width 0.4) (layer "F.Cu") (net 2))
 (segment locked (start 158.24 100.38) (end 156.24 100.38) (width 0.4) (layer "F.Cu") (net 2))
 (segment locked (start 158.8 100.94) (end 158.24 100.38) (width 0.4) (layer "F.Cu") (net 2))
 (segment locked (start 134.607677 114.825) (end 134.607677 107.332323) (width 0.8) (layer "F.Cu") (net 2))
 (segment locked (start 152.24 100.38) (end 156.24 100.38) (width 0.4) (layer "F.Cu") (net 2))
 (segment locked (start 160.91 106.71) (end 159.57 106.71) (width 0.4) (layer "F.Cu") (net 2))
 (segment locked (start 138.74 74.825) (end 139.3025 75.3875) (width 0.4) (layer "F.Cu") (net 2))
 (segment locked (start 129.717 77.197) (end 132.089 74.825) (width 0.4) (layer "F.Cu") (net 2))
 (segment locked (start 168 95.725) (end 166.185 97.54) (width 0.4) (layer "F.Cu") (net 2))
 (segment locked (start 162 102.525) (end 162.8 102.525) (width 0.4) (layer "F.Cu") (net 2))
 (segment locked (start 158.8 102.525) (end 158.8 100.94) (width 0.4) (layer "F.Cu") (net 2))
 (segment locked (start 140.365 75.7625) (end 144.24 75.7625) (width 0.4) (layer "F.Cu") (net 2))
 (segment locked (start 145.74 91.825) (end 146.4 92.485) (width 0.4) (layer "F.Cu") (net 2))
 (segment locked (start 117.144 77.197) (end 117.144 92.945) (width 0.4) (layer "F.Cu") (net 2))
 (segment locked (start 136.24 79.7625) (end 140.74 79.7625) (width 0.4) (layer "F.Cu") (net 2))
 (segment locked (start 140.74 91.825) (end 145.74 91.825) (width 0.4) (layer "F.Cu") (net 2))
 (segment locked (start 134.24 81.325) (end 133.26 82.305) (width 0.4) (layer "F.Cu") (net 8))
 (segment locked (start 133.26 82.305) (end 132.24 82.305) (width 0.4) (layer "F.Cu") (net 8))
 (segment locked (start 146.69 81.325) (end 144.24 81.325) (width 0.4) (layer "F.Cu") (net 8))
 (segment locked (start 144.24 81.325) (end 134.24 81.325) (width 0.4) (layer "F.Cu") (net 8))
 (segment locked (start 144.24 78.8875) (end 144.24 81.325) (width 0.4) (layer "F.Cu") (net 8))
 (segment locked (start 132.26 82.325) (end 132.24 82.305) (width 0.4) (layer "F.Cu") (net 8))
 (segment locked (start 140.74 84.825) (end 146.19 84.825) (width 0.4) (layer "F.Cu") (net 11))
 (segment locked (start 146.19 84.825) (end 146.69 85.325) (width 0.4) (layer "F.Cu") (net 11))
 (segment locked (start 140.74 82.8875) (end 140.74 84.825) (width 0.4) (layer "F.Cu") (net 11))
 (segment locked (start 132.214237 84.825) (end 140.74 84.825) (width 0.4) (layer "F.Cu") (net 11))
 (segment locked (start 143.24 89.325) (end 141.24 89.325) (width 0.4) (layer "F.Cu") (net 10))
 (segment locked (start 136.1775 76.825) (end 136.1775 76.8875) (width 0.4) (layer "F.Cu") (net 10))
 (segment locked (start 128.74 81.825) (end 128.74 86.825) (width 0.4) (layer "F.Cu") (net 10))
 (segment locked (start 136.1775 76.8875) (end 133.28 79.785) (width 0.4) (layer "F.Cu") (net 10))
 (segment locked (start 139.24 91.325) (end 133.24 91.325) (width 0.4) (layer "F.Cu") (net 10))
 (segment locked (start 132.24 79.785) (end 131.946796 79.785) (width 0.4) (layer "F.Cu") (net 10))
 (segment locked (start 143.74 89.825) (end 143.24 89.325) (width 0.4) (layer "F.Cu") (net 10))
 (segment locked (start 147.24 89.825) (end 143.74 89.825) (width 0.4) (layer "F.Cu") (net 10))
 (segment locked (start 133.24 91.325) (end 128.74 86.825) (width 0.4) (layer "F.Cu") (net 10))
 (segment locked (start 131.946796 79.785) (end 131.906796 79.825) (width 0.4) (layer "F.Cu") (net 10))
 (segment locked (start 130.74 79.825) (end 128.74 81.825) (width 0.4) (layer "F.Cu") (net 10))
 (segment locked (start 133.28 79.785) (end 132.24 79.785) (width 0.4) (layer "F.Cu") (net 10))
 (segment locked (start 141.24 89.325) (end 139.24 91.325) (width 0.4) (layer "F.Cu") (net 10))
 (segment locked (start 148 90.585) (end 147.24 89.825) (width 0.4) (layer "F.Cu") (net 10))
 (segment locked (start 131.906796 79.825) (end 130.74 79.825) (width 0.4) (layer "F.Cu") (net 10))
 (segment locked (start 148 94.325) (end 148 90.585) (width 0.4) (layer "F.Cu") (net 10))
 (segment locked (start 143.14 86.325) (end 143.24 86.225) (width 0.4) (layer "F.Cu") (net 1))
 (segment locked (start 130.24 86.325) (end 137.74 86.325) (width 0.4) (layer "F.Cu") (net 1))
 (segment locked (start 137.74 86.325) (end 143.14 86.325) (width 0.4) (layer "F.Cu") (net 1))
 (segment locked (start 135.5625 83.565) (end 132.24 83.565) (width 0.4) (layer "F.Cu") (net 1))
 (segment locked (start 130.5 83.565) (end 132.24 83.565) (width 0.4) (layer "F.Cu") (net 1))
 (segment locked (start 136.24 82.8875) (end 135.5625 83.565) (width 0.4) (layer "F.Cu") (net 1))
 (segment locked (start 130.24 83.825) (end 130.5 83.565) (width 0.4) (layer "F.Cu") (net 1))
 (segment locked (start 130.24 86.325) (end 130.24 83.825) (width 0.4) (layer "F.Cu") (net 1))
 (segment locked (start 149.2 102.525) (end 149.2 110.825) (width 0.4) (layer "F.Cu") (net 3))
 (segment locked (start 149.2 110.825) (end 151.95 113.575) (width 0.4) (layer "F.Cu") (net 3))
 (segment locked (start 151.95 113.575) (end 151.435 113.575) (width 0.4) (layer "F.Cu") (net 3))
 (segment locked (start 151.95 113.575) (end 149.74 111.365) (width 1.2) (layer "F.Cu") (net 3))
 (segment locked (start 149.74 111.365) (end 149.74 111.325) (width 1.2) (layer "F.Cu") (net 3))
 (segment locked (start 157.03 111.535) (end 157.2 111.365) (width 1.2) (layer "F.Cu") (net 5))
 (segment locked (start 157.03 113.575) (end 157.03 111.535) (width 1.2) (layer "F.Cu") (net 5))
 (segment locked (start 157.2 102.525) (end 157.2 111.365) (width 0.4) (layer "F.Cu") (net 5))
 (segment locked (start 158 108.085) (end 159.57 109.655) (width 0.4) (layer "F.Cu") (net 6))
 (segment locked (start 159.57 113.575) (end 159.57 111.155) (width 1.2) (layer "F.Cu") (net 6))
 (segment locked (start 159.57 109.655) (end 159.57 111.155) (width 0.4) (layer "F.Cu") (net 6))
 (segment locked (start 158 102.525) (end 158 108.085) (width 0.4) (layer "F.Cu") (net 6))
 (segment locked (start 154.49 113.575) (end 154.49 111.075) (width 1.2) (layer "F.Cu") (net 4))
 (segment locked (start 150 106.085) (end 154.49 110.575) (width 0.4) (layer "F.Cu") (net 4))
 (segment locked (start 154.49 110.575) (end 154.49 111.075) (width 0.4) (layer "F.Cu") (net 4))
 (segment locked (start 150 102.525) (end 150 106.085) (width 0.4) (layer "F.Cu") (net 4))
 (segment locked (start 139.34 87.825) (end 146.74 87.825) (width 0.4) (layer "F.Cu") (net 13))
 (segment locked (start 146.74 87.825) (end 148.8 89.885) (width 0.4) (layer "F.Cu") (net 13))
 (segment locked (start 137.74 89.425) (end 139.34 87.825) (width 0.4) (layer "F.Cu") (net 13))
 (segment locked (start 148.8 89.885) (end 148.8 94.325) (width 0.4) (layer "F.Cu") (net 13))
 (segment locked (start 149.6 94.325) (end 149.6 85.515) (width 0.4) (layer "F.Cu") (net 19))
 (segment locked (start 149.6 85.515) (end 149.79 85.325) (width 0.4) (layer "F.Cu") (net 19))
 (segment locked (start 152.24 83.325) (end 150.24 81.325) (width 0.4) (layer "F.Cu") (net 9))
 (segment locked (start 152.24 88.325) (end 152.24 83.325) (width 0.4) (layer "F.Cu") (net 9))
 (segment locked (start 150.24 81.325) (end 149.79 81.325) (width 0.4) (layer "F.Cu") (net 9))
 (segment locked (start 150.4 94.325) (end 150.4 90.165) (width 0.4) (layer "F.Cu") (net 9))
 (segment locked (start 150.4 90.165) (end 152.24 88.325) (width 0.4) (layer "F.Cu") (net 9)))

